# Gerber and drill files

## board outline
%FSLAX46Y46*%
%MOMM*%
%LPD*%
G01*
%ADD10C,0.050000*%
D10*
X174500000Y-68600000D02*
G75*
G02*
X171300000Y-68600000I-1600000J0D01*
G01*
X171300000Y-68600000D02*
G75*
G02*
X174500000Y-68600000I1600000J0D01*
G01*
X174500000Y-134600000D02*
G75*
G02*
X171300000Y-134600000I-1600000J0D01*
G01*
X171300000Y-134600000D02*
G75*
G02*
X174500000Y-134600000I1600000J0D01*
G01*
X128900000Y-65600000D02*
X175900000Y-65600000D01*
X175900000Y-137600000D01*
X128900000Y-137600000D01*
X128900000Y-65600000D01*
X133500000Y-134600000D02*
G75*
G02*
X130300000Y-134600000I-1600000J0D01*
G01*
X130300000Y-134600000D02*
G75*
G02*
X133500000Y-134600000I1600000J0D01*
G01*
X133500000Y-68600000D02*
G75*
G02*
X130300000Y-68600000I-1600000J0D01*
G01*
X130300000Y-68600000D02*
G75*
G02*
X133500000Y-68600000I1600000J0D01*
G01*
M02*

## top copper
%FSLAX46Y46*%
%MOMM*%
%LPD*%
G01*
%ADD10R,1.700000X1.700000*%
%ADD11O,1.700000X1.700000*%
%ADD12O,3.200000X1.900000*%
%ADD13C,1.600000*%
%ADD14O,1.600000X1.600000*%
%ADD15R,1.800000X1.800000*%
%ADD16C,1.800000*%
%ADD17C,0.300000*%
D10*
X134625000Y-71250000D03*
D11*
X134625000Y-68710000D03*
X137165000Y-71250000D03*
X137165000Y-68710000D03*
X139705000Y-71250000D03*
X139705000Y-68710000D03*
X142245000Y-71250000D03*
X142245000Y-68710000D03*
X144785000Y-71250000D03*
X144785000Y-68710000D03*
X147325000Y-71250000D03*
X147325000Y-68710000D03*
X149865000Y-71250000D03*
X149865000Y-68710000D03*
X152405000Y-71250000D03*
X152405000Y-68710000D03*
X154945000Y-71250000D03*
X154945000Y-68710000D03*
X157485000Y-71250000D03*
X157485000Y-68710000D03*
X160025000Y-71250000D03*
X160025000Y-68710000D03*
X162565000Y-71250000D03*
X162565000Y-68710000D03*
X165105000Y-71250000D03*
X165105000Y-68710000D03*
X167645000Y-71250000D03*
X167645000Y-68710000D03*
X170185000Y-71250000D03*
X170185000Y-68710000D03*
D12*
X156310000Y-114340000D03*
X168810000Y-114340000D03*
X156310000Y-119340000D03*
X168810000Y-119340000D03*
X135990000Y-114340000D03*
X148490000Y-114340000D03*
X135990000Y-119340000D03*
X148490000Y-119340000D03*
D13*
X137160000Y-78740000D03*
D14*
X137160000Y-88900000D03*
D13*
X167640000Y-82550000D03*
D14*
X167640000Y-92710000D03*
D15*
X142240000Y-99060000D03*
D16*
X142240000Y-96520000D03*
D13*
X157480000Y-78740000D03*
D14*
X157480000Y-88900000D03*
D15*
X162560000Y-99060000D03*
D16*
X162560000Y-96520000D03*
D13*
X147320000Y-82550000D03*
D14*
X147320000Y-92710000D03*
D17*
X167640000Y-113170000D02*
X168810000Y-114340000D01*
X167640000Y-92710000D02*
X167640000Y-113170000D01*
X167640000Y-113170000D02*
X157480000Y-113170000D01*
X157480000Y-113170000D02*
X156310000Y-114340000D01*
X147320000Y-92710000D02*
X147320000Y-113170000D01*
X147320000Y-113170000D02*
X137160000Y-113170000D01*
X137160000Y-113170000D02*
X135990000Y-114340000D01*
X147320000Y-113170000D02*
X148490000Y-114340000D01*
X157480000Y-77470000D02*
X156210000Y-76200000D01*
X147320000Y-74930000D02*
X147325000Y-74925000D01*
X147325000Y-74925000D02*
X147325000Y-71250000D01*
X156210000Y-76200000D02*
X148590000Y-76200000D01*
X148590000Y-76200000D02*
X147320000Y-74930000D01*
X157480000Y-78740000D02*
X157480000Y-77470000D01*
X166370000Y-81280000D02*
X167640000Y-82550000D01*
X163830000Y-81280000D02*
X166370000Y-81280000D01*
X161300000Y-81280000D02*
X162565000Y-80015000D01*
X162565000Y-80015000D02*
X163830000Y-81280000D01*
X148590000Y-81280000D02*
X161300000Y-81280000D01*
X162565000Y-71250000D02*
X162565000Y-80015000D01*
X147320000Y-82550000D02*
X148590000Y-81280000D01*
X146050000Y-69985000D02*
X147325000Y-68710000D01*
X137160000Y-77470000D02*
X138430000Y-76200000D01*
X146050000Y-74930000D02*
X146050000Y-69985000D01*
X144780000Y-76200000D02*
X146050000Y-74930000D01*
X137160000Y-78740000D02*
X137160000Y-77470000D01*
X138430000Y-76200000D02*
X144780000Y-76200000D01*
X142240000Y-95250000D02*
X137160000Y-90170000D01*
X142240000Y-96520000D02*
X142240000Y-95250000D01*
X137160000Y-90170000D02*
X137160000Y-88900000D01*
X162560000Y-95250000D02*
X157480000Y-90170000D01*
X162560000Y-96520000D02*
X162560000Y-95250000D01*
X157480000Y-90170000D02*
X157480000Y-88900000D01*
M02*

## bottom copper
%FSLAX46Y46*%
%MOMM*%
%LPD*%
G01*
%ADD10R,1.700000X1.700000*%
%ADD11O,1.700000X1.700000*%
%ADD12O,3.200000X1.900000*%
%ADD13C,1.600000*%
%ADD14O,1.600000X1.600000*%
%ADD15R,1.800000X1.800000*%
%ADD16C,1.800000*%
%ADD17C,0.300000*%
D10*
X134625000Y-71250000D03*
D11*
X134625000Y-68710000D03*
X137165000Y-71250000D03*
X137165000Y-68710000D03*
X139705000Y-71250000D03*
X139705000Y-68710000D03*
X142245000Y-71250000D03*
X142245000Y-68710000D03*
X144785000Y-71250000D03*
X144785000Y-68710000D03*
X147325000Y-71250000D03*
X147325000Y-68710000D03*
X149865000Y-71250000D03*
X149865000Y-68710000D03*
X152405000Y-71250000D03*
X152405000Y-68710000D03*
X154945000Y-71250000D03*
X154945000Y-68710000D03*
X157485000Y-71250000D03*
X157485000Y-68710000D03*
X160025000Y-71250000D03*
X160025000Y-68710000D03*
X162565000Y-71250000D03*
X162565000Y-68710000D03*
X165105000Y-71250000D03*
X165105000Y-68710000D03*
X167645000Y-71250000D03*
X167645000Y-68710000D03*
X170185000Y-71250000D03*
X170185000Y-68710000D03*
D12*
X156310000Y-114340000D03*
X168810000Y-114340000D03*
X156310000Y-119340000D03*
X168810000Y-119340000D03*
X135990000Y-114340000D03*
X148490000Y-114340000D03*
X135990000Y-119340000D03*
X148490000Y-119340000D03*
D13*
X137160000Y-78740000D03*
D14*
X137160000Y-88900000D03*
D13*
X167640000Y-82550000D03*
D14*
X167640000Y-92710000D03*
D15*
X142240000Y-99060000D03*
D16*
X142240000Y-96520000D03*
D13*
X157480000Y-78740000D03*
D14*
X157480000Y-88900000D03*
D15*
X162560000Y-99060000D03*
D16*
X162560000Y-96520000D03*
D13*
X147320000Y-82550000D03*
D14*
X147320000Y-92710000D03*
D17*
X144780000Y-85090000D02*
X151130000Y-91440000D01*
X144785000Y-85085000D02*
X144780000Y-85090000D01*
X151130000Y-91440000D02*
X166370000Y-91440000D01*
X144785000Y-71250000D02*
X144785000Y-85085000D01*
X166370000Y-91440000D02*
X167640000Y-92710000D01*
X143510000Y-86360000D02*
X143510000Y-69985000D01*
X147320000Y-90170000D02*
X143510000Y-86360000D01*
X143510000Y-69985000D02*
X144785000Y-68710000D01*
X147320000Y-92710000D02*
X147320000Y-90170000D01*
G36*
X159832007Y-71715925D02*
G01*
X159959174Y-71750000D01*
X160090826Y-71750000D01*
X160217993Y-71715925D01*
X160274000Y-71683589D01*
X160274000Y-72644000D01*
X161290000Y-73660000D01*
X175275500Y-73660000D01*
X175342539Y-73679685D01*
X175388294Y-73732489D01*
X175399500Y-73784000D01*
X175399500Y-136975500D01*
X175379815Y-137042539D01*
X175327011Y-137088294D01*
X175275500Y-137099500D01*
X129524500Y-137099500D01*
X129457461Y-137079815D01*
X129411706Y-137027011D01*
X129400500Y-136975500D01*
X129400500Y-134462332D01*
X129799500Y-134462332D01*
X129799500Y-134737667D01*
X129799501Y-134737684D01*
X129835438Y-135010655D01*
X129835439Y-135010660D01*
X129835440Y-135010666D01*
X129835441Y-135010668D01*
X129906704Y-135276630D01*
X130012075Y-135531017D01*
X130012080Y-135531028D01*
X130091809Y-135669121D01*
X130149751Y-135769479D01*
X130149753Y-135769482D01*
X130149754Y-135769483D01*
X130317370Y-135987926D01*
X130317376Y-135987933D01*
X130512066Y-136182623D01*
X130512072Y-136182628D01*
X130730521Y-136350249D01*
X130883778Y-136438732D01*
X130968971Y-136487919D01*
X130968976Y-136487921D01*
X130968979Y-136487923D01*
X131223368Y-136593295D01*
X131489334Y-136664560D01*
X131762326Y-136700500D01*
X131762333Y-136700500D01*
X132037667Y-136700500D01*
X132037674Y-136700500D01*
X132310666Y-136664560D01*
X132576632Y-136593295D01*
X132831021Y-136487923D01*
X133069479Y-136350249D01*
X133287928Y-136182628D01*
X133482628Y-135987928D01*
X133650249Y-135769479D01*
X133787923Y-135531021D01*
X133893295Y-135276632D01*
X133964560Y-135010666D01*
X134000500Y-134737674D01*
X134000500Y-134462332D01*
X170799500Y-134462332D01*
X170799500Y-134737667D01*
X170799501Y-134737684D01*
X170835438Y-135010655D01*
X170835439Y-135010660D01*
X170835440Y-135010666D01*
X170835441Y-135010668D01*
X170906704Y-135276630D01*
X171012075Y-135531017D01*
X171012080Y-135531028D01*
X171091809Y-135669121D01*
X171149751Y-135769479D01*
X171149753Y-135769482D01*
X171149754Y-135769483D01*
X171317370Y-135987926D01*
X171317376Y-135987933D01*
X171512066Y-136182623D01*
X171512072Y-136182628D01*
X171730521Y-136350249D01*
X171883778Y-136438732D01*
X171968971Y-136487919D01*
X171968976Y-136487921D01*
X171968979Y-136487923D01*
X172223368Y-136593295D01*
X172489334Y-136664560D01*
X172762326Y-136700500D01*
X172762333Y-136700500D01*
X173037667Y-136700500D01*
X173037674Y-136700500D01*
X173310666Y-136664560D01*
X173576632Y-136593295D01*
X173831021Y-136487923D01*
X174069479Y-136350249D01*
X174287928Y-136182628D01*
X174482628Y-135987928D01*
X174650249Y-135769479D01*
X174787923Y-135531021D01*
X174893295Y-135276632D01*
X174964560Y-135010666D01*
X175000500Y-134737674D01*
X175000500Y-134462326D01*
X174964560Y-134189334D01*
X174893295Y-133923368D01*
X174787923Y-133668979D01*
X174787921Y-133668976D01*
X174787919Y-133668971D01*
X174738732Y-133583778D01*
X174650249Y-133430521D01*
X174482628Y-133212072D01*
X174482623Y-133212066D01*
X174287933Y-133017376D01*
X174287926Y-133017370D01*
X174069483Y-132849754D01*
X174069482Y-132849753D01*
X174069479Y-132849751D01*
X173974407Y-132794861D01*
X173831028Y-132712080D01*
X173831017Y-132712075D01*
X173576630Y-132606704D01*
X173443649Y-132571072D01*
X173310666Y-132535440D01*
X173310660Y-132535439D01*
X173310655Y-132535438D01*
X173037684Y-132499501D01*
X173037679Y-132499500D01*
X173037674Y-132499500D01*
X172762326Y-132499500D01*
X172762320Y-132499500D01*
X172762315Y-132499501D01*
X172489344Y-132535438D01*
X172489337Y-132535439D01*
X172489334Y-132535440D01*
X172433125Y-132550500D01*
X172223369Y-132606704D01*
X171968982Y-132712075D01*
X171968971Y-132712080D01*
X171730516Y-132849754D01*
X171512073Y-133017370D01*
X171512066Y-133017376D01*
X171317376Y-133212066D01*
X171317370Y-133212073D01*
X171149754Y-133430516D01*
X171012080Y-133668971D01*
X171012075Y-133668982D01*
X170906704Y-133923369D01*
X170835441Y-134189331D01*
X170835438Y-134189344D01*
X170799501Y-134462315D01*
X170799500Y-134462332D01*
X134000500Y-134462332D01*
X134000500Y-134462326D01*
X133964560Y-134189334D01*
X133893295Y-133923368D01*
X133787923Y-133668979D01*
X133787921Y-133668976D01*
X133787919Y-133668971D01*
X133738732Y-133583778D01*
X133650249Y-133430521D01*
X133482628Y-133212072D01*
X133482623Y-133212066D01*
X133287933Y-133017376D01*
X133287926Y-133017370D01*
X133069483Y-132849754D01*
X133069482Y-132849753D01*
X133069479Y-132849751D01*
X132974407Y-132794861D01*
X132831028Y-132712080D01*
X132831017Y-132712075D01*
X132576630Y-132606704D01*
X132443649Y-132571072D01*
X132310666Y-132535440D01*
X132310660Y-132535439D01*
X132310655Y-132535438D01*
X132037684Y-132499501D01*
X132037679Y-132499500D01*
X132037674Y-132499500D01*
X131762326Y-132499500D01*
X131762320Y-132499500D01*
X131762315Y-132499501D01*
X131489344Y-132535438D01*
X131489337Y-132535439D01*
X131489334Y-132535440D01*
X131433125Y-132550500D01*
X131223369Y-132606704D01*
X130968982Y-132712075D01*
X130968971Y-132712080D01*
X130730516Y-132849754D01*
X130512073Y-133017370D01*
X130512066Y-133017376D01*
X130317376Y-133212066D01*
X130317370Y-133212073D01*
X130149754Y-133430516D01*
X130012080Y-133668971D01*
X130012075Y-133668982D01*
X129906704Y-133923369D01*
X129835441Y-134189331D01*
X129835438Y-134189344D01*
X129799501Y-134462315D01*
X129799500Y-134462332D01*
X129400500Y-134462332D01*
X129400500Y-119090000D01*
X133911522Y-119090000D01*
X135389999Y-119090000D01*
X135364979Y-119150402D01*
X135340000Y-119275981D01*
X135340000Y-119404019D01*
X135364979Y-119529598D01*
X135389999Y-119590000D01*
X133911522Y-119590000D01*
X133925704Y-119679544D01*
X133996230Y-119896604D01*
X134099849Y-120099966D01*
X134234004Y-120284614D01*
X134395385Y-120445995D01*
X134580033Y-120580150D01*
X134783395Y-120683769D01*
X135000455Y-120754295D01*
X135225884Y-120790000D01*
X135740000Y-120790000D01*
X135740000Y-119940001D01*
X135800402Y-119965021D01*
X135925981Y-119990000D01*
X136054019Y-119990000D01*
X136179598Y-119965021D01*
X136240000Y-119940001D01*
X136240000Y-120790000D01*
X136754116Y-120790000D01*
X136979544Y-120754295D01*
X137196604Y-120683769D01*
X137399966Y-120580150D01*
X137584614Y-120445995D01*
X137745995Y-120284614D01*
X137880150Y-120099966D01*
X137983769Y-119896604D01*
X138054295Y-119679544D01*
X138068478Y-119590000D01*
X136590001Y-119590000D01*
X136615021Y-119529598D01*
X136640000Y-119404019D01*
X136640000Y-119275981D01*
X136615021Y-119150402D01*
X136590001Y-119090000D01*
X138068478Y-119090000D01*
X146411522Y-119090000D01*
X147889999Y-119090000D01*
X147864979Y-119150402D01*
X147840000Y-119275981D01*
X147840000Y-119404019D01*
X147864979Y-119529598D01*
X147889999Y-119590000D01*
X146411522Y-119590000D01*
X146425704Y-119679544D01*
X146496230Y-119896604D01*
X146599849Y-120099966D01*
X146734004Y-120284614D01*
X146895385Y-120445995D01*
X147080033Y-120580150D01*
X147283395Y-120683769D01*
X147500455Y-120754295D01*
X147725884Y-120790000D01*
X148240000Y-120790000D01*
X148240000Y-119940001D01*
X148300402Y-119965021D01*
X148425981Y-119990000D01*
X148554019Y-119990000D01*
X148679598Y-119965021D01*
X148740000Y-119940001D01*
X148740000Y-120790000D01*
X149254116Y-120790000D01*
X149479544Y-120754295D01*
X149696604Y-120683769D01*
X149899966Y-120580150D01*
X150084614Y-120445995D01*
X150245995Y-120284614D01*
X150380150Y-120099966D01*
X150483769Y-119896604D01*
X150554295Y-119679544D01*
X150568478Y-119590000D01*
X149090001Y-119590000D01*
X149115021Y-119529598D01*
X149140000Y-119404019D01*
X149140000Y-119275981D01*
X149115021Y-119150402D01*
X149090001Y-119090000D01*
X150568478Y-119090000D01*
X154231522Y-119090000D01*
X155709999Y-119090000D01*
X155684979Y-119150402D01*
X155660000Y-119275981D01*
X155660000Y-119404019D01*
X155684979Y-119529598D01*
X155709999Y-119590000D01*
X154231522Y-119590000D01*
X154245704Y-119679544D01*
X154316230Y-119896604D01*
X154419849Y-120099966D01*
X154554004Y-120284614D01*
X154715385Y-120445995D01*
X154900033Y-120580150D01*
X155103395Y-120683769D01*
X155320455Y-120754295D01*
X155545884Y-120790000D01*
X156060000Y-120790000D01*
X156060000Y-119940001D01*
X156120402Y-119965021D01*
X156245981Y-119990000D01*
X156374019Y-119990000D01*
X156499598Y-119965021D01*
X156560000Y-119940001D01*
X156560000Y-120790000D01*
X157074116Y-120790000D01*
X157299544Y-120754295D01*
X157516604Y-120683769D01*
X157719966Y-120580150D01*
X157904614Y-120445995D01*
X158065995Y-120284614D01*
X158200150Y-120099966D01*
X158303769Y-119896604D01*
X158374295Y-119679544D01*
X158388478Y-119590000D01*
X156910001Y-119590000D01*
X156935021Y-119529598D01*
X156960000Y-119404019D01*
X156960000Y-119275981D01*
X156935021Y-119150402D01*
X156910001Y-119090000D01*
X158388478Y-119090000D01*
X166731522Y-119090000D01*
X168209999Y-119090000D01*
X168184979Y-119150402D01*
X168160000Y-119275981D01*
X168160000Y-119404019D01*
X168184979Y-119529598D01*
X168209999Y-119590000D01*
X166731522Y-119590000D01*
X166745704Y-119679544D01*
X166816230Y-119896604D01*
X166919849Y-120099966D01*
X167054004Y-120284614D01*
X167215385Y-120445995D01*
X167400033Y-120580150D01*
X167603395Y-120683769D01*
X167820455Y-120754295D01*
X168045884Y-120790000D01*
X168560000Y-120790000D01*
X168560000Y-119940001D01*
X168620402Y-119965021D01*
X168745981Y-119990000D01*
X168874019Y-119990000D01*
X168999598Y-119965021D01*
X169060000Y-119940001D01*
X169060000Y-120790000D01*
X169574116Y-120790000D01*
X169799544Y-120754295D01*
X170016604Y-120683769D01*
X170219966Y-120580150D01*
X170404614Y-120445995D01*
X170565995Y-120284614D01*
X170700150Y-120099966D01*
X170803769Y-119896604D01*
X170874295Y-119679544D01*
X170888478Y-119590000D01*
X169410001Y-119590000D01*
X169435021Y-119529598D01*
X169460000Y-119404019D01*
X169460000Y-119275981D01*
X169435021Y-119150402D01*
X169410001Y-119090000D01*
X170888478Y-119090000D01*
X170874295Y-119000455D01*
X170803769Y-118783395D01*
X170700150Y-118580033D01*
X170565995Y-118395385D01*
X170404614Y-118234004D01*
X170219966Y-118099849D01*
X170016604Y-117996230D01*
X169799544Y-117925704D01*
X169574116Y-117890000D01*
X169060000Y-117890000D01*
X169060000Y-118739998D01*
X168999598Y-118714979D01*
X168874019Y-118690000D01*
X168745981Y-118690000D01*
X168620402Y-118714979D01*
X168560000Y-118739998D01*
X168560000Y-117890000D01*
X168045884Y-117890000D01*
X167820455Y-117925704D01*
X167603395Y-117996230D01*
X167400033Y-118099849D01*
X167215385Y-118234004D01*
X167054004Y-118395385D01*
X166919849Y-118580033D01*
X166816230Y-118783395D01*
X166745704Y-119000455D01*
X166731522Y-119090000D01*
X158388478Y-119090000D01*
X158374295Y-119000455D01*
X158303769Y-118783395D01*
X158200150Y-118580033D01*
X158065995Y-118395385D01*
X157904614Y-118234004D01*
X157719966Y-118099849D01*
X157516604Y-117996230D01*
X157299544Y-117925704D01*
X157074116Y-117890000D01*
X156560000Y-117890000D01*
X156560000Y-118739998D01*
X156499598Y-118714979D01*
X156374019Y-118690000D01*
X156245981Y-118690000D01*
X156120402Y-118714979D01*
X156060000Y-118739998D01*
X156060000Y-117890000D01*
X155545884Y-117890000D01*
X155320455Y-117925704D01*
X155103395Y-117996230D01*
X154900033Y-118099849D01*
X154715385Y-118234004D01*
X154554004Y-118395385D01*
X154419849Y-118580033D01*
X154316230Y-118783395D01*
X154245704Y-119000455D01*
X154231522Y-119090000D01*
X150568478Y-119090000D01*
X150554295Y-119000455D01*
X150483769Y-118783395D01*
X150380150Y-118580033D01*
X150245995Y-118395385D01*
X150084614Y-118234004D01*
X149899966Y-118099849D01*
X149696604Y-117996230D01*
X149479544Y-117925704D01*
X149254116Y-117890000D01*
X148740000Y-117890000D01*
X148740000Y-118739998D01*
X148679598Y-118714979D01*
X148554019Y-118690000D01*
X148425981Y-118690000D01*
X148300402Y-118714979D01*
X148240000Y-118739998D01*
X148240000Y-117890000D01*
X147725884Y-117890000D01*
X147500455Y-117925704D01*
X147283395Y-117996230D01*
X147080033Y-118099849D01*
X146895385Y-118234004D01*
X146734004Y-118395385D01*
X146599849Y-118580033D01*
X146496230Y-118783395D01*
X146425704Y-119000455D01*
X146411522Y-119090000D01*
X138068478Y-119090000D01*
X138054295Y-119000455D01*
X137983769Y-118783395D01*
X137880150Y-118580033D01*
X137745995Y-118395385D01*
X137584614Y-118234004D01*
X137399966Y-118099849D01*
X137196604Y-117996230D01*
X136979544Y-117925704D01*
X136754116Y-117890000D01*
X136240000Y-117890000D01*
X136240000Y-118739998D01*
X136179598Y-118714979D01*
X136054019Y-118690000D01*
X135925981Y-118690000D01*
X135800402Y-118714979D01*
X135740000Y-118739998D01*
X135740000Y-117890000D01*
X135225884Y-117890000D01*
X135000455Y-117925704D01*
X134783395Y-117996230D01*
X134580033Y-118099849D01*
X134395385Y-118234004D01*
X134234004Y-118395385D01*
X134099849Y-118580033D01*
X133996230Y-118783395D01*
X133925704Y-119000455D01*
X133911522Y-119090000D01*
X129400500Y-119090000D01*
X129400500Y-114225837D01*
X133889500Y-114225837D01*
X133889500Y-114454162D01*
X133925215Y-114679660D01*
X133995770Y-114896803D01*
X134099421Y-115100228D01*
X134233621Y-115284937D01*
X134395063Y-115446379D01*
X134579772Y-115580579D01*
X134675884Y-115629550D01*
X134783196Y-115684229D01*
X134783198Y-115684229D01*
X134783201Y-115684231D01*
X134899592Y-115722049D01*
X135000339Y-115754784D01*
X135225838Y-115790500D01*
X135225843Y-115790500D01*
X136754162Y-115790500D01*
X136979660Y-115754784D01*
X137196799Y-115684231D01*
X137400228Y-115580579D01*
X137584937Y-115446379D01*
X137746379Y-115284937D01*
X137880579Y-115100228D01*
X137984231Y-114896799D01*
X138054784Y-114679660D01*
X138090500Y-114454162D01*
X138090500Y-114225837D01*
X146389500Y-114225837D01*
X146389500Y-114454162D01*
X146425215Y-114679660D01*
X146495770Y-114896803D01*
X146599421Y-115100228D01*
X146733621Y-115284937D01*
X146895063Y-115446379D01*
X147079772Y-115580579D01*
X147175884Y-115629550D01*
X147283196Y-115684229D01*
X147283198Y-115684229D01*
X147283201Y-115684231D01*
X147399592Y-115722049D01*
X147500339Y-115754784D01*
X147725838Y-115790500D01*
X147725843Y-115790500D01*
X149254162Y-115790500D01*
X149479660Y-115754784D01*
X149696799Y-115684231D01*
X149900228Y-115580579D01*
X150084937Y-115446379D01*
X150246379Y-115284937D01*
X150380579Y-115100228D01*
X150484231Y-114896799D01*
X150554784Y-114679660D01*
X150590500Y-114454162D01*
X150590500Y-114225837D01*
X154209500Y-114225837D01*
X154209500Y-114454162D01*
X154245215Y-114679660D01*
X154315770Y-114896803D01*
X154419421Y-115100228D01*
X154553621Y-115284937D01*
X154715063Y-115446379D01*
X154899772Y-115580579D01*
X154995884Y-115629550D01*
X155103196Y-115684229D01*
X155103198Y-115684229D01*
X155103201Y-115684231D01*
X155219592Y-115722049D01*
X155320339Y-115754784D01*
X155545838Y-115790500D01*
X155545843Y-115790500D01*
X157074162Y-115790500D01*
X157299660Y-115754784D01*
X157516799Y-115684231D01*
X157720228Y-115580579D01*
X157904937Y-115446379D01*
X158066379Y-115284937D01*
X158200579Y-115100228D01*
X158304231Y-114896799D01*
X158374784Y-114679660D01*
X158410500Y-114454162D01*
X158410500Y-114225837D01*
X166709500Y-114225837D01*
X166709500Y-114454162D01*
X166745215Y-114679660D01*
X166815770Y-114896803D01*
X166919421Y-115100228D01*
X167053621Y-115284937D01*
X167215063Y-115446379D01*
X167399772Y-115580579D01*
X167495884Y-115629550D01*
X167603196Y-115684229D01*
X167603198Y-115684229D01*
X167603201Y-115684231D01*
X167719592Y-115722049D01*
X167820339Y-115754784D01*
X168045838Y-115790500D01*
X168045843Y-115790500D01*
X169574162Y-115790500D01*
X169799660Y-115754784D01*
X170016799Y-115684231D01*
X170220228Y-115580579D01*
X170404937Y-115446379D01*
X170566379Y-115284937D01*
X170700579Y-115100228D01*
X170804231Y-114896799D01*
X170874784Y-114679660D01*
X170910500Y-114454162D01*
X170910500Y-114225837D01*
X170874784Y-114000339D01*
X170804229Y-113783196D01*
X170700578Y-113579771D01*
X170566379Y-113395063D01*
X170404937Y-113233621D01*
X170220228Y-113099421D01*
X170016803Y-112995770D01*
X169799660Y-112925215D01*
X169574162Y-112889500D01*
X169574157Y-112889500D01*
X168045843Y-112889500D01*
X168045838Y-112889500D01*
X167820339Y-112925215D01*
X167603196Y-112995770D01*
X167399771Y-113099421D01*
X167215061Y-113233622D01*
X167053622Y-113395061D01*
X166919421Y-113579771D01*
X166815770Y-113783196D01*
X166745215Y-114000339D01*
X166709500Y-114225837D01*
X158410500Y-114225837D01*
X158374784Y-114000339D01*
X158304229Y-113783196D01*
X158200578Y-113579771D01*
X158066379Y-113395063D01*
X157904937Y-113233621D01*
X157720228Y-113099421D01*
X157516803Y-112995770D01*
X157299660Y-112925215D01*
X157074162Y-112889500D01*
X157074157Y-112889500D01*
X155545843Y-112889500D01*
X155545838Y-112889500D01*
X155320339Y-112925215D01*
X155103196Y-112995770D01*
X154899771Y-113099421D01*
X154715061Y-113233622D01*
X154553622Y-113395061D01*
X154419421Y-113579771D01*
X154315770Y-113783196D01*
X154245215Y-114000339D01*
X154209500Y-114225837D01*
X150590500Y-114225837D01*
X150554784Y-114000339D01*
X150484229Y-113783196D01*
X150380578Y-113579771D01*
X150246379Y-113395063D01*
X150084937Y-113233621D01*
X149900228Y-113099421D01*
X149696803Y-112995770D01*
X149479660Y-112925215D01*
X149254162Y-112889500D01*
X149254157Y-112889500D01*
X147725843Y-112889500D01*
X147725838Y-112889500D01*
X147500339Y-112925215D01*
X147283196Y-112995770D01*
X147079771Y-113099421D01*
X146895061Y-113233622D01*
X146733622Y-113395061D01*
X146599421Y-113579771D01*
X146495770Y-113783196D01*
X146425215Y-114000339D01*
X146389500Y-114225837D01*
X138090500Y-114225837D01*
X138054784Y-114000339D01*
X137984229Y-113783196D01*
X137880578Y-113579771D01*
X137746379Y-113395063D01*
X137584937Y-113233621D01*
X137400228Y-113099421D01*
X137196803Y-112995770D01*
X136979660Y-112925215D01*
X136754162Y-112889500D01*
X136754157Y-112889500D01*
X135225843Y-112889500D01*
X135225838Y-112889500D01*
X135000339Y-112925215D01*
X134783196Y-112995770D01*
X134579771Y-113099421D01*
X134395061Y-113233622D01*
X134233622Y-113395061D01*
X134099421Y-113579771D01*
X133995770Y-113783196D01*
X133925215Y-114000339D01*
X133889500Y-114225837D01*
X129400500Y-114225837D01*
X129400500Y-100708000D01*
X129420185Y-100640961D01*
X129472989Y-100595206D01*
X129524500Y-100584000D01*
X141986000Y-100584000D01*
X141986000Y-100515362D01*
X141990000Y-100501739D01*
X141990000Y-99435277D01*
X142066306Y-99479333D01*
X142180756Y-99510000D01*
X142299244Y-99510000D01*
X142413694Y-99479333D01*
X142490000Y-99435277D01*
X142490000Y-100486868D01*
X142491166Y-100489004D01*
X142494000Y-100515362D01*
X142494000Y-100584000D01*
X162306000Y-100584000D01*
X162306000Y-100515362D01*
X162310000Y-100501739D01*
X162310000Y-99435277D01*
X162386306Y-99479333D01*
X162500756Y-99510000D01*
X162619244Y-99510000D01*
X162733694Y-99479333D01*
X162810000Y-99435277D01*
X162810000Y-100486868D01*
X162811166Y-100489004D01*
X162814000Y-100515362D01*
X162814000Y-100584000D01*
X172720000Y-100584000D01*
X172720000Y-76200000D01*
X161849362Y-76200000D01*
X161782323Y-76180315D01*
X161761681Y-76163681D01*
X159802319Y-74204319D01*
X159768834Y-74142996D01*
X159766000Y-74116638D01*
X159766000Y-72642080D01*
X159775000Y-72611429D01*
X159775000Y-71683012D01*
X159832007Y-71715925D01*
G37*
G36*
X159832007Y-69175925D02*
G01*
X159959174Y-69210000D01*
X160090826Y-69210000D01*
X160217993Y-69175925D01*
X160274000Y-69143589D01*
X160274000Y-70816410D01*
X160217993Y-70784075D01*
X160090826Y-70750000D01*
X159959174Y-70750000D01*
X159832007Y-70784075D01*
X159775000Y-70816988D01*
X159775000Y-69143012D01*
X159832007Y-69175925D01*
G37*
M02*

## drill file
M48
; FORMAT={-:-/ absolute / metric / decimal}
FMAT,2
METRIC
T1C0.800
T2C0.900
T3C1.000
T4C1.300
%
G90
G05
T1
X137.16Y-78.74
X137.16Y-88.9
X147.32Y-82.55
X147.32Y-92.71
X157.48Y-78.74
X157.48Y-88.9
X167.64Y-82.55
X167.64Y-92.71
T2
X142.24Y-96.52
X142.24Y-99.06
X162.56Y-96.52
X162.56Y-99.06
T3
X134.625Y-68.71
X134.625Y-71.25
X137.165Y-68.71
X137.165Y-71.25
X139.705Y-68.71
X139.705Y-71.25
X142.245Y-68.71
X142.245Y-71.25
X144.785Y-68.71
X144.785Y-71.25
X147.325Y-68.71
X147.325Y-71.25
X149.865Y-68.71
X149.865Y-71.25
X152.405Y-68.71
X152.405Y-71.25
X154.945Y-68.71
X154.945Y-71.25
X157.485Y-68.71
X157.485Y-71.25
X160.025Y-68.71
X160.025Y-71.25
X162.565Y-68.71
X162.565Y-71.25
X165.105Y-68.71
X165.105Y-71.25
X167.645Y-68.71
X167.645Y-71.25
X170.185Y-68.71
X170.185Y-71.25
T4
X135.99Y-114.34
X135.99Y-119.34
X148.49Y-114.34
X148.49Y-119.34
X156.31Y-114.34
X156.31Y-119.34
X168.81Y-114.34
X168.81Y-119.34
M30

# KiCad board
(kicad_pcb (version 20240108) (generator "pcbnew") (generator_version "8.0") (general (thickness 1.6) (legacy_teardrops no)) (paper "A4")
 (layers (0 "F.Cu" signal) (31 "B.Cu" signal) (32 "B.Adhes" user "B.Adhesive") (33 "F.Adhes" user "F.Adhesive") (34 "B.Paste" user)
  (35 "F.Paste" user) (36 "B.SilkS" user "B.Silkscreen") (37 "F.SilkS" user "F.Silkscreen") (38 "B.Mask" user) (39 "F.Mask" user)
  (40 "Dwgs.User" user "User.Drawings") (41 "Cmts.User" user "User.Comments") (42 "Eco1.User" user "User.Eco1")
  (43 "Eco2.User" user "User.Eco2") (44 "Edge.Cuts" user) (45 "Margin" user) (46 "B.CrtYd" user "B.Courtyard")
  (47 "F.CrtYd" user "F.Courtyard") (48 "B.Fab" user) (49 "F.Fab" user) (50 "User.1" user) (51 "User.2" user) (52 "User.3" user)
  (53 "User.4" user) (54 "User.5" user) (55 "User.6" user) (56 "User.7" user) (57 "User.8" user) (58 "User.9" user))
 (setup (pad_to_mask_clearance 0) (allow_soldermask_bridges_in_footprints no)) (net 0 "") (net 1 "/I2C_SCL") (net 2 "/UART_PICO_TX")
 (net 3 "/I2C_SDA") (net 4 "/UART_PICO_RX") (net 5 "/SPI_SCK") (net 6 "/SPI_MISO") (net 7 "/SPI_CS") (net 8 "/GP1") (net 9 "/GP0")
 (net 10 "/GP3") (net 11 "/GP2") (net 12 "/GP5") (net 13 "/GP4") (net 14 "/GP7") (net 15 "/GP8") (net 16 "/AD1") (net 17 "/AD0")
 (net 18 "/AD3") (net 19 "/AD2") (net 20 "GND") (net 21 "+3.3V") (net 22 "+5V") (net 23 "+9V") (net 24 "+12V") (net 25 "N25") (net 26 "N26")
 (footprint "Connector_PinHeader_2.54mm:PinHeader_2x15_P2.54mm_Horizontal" (layer "F.Cu") (at 134.625 71.25 90)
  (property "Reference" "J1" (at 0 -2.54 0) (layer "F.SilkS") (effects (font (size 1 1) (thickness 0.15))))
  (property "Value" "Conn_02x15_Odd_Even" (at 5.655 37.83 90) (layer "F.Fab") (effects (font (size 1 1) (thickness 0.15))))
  (pad "1" thru_hole rect (at 0 0 90) (size 1.7 1.7) (drill 1) (layers "*.Cu" "*.Mask") (remove_unused_layers no) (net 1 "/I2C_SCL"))
  (pad "2" thru_hole oval (at 2.54 0 90) (size 1.7 1.7) (drill 1) (layers "*.Cu" "*.Mask") (remove_unused_layers no) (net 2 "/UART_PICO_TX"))
  (pad "3" thru_hole oval (at 0 2.54 90) (size 1.7 1.7) (drill 1) (layers "*.Cu" "*.Mask") (remove_unused_layers no) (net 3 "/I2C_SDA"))
  (pad "4" thru_hole oval (at 2.54 2.54 90) (size 1.7 1.7) (drill 1) (layers "*.Cu" "*.Mask") (remove_unused_layers no)
   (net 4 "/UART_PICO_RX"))
  (pad "5" thru_hole oval (at 0 5.08 90) (size 1.7 1.7) (drill 1) (layers "*.Cu" "*.Mask") (remove_unused_layers no) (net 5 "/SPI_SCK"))
  (pad "6" thru_hole oval (at 2.54 5.08 90) (size 1.7 1.7) (drill 1) (layers "*.Cu" "*.Mask") (remove_unused_layers no) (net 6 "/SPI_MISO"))
  (pad "7" thru_hole oval (at 0 7.62 90) (size 1.7 1.7) (drill 1) (layers "*.Cu" "*.Mask") (remove_unused_layers no) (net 6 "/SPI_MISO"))
  (pad "8" thru_hole oval (at 2.54 7.62 90) (size 1.7 1.7) (drill 1) (layers "*.Cu" "*.Mask") (remove_unused_layers no) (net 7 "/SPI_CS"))
  (pad "9" thru_hole oval (at 0 10.16 90) (size 1.7 1.7) (drill 1) (layers "*.Cu" "*.Mask") (remove_unused_layers no) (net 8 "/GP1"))
  (pad "10" thru_hole oval (at 2.54 10.16 90) (size 1.7 1.7) (drill 1) (layers "*.Cu" "*.Mask") (remove_unused_layers no) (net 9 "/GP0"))
  (pad "11" thru_hole oval (at 0 12.7 90) (size 1.7 1.7) (drill 1) (layers "*.Cu" "*.Mask") (remove_unused_layers no) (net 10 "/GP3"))
  (pad "12" thru_hole oval (at 2.54 12.7 90) (size 1.7 1.7) (drill 1) (layers "*.Cu" "*.Mask") (remove_unused_layers no) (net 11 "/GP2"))
  (pad "13" thru_hole oval (at 0 15.24 90) (size 1.7 1.7) (drill 1) (layers "*.Cu" "*.Mask") (remove_unused_layers no) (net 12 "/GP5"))
  (pad "14" thru_hole oval (at 2.54 15.24 90) (size 1.7 1.7) (drill 1) (layers "*.Cu" "*.Mask") (remove_unused_layers no) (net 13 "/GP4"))
  (pad "15" thru_hole oval (at 0 17.78 90) (size 1.7 1.7) (drill 1) (layers "*.Cu" "*.Mask") (remove_unused_layers no) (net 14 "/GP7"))
  (pad "16" thru_hole oval (at 2.54 17.78 90) (size 1.7 1.7) (drill 1) (layers "*.Cu" "*.Mask") (remove_unused_layers no) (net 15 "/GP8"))
  (pad "17" thru_hole oval (at 0 20.32 90) (size 1.7 1.7) (drill 1) (layers "*.Cu" "*.Mask") (remove_unused_layers no) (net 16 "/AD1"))
  (pad "18" thru_hole oval (at 2.54 20.32 90) (size 1.7 1.7) (drill 1) (layers "*.Cu" "*.Mask") (remove_unused_layers no) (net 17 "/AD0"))
  (pad "19" thru_hole oval (at 0 22.86 90) (size 1.7 1.7) (drill 1) (layers "*.Cu" "*.Mask") (remove_unused_layers no) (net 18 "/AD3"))
  (pad "20" thru_hole oval (at 2.54 22.86 90) (size 1.7 1.7) (drill 1) (layers "*.Cu" "*.Mask") (remove_unused_layers no) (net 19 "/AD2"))
  (pad "21" thru_hole oval (at 0 25.4 90) (size 1.7 1.7) (drill 1) (layers "*.Cu" "*.Mask") (remove_unused_layers no) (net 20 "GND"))
  (pad "22" thru_hole oval (at 2.54 25.4 90) (size 1.7 1.7) (drill 1) (layers "*.Cu" "*.Mask") (remove_unused_layers no) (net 20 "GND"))
  (pad "23" thru_hole oval (at 0 27.94 90) (size 1.7 1.7) (drill 1) (layers "*.Cu" "*.Mask") (remove_unused_layers no) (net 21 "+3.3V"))
  (pad "24" thru_hole oval (at 2.54 27.94 90) (size 1.7 1.7) (drill 1) (layers "*.Cu" "*.Mask") (remove_unused_layers no) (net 21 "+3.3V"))
  (pad "25" thru_hole oval (at 0 30.48 90) (size 1.7 1.7) (drill 1) (layers "*.Cu" "*.Mask") (remove_unused_layers no) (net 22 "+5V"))
  (pad "26" thru_hole oval (at 2.54 30.48 90) (size 1.7 1.7) (drill 1) (layers "*.Cu" "*.Mask") (remove_unused_layers no) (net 22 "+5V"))
  (pad "27" thru_hole oval (at 0 33.02 90) (size 1.7 1.7) (drill 1) (layers "*.Cu" "*.Mask") (remove_unused_layers no) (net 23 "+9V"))
  (pad "28" thru_hole oval (at 2.54 33.02 90) (size 1.7 1.7) (drill 1) (layers "*.Cu" "*.Mask") (remove_unused_layers no) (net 23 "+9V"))
  (pad "29" thru_hole oval (at 0 35.56 90) (size 1.7 1.7) (drill 1) (layers "*.Cu" "*.Mask") (remove_unused_layers no) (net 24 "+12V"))
  (pad "30" thru_hole oval (at 2.54 35.56 90) (size 1.7 1.7) (drill 1) (layers "*.Cu" "*.Mask") (remove_unused_layers no) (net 24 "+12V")))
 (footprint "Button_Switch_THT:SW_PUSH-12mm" (layer "F.Cu") (at 156.31 114.34)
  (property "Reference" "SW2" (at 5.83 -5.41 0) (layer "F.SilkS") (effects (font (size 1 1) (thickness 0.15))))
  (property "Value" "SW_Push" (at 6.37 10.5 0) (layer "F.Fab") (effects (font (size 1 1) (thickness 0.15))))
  (pad "1" thru_hole oval (at 0 0) (size 3.2 1.9) (drill 1.3) (layers "*.Cu" "*.Mask") (remove_unused_layers no) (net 8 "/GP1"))
  (pad "1" thru_hole oval (at 12.5 0) (size 3.2 1.9) (drill 1.3) (layers "*.Cu" "*.Mask") (remove_unused_layers no) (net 8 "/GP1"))
  (pad "2" thru_hole oval (at 0 5) (size 3.2 1.9) (drill 1.3) (layers "*.Cu" "*.Mask") (remove_unused_layers no) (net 20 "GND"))
  (pad "2" thru_hole oval (at 12.5 5) (size 3.2 1.9) (drill 1.3) (layers "*.Cu" "*.Mask") (remove_unused_layers no) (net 20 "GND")))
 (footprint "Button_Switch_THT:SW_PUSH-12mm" (layer "F.Cu") (at 135.99 114.34)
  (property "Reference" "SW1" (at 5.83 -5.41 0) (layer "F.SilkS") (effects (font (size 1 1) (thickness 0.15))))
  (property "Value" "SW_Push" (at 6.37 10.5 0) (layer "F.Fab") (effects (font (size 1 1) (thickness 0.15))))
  (pad "1" thru_hole oval (at 0 0) (size 3.2 1.9) (drill 1.3) (layers "*.Cu" "*.Mask") (remove_unused_layers no) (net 9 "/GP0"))
  (pad "1" thru_hole oval (at 12.5 0) (size 3.2 1.9) (drill 1.3) (layers "*.Cu" "*.Mask") (remove_unused_layers no) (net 9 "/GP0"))
  (pad "2" thru_hole oval (at 0 5) (size 3.2 1.9) (drill 1.3) (layers "*.Cu" "*.Mask") (remove_unused_layers no) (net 20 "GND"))
  (pad "2" thru_hole oval (at 12.5 5) (size 3.2 1.9) (drill 1.3) (layers "*.Cu" "*.Mask") (remove_unused_layers no) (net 20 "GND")))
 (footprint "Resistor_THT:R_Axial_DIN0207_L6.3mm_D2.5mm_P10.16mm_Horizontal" (layer "F.Cu") (at 137.16 78.74 -90)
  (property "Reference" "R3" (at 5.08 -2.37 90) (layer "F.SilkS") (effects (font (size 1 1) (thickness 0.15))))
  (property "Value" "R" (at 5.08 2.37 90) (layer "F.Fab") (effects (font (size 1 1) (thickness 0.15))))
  (pad "1" thru_hole circle (at 0 0 270) (size 1.6 1.6) (drill 0.8) (layers "*.Cu" "*.Mask") (remove_unused_layers no) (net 11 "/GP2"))
  (pad "2" thru_hole oval (at 10.16 0 270) (size 1.6 1.6) (drill 0.8) (layers "*.Cu" "*.Mask") (remove_unused_layers no) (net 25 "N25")))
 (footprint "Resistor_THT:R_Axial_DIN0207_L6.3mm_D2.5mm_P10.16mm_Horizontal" (layer "F.Cu") (at 167.64 82.55 -90)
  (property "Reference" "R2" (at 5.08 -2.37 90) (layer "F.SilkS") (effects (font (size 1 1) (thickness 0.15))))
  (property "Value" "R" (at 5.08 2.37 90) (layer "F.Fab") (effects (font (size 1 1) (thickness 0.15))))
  (pad "1" thru_hole circle (at 0 0 270) (size 1.6 1.6) (drill 0.8) (layers "*.Cu" "*.Mask") (remove_unused_layers no) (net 21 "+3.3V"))
  (pad "2" thru_hole oval (at 10.16 0 270) (size 1.6 1.6) (drill 0.8) (layers "*.Cu" "*.Mask") (remove_unused_layers no) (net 8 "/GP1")))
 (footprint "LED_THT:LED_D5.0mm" (layer "F.Cu") (at 142.24 99.06 90)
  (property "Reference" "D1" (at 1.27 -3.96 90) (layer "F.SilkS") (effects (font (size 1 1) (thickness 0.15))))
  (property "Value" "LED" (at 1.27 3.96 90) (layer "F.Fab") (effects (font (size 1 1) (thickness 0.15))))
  (pad "1" thru_hole rect (at 0 0 90) (size 1.8 1.8) (drill 0.9) (layers "*.Cu" "*.Mask") (remove_unused_layers no) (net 20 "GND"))
  (pad "2" thru_hole circle (at 2.54 0 90) (size 1.8 1.8) (drill 0.9) (layers "*.Cu" "*.Mask") (remove_unused_layers no) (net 25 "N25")))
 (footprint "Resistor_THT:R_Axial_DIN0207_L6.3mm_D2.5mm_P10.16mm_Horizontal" (layer "F.Cu") (at 157.48 78.74 -90)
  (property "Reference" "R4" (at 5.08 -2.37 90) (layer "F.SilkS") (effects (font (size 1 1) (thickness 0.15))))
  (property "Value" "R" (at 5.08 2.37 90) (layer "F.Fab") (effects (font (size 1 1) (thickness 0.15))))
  (pad "1" thru_hole circle (at 0 0 270) (size 1.6 1.6) (drill 0.8) (layers "*.Cu" "*.Mask") (remove_unused_layers no) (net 10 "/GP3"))
  (pad "2" thru_hole oval (at 10.16 0 270) (size 1.6 1.6) (drill 0.8) (layers "*.Cu" "*.Mask") (remove_unused_layers no) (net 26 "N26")))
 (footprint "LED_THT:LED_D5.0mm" (layer "F.Cu") (at 162.56 99.06 90)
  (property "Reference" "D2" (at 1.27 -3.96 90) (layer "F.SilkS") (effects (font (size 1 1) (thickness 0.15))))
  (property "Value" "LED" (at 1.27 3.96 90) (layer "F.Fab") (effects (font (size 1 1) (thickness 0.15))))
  (pad "1" thru_hole rect (at 0 0 90) (size 1.8 1.8) (drill 0.9) (layers "*.Cu" "*.Mask") (remove_unused_layers no) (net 20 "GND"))
  (pad "2" thru_hole circle (at 2.54 0 90) (size 1.8 1.8) (drill 0.9) (layers "*.Cu" "*.Mask") (remove_unused_layers no) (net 26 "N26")))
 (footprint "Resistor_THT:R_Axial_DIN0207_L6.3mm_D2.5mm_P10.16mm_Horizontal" (layer "F.Cu") (at 147.32 82.55 -90)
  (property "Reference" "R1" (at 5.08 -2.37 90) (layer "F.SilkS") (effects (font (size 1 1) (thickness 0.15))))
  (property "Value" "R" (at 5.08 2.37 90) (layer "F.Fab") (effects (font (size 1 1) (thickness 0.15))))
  (pad "1" thru_hole circle (at 0 0 270) (size 1.6 1.6) (drill 0.8) (layers "*.Cu" "*.Mask") (remove_unused_layers no) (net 21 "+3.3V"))
  (pad "2" thru_hole oval (at 10.16 0 270) (size 1.6 1.6) (drill 0.8) (layers "*.Cu" "*.Mask") (remove_unused_layers no) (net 9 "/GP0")))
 (gr_circle (center 172.9 68.6) (end 172.9 70.2) (stroke (width 0.05) (type default)) (fill none) (layer "Edge.Cuts"))
 (gr_circle (center 172.9 134.6) (end 171.3 134.6) (stroke (width 0.05) (type default)) (fill none) (layer "Edge.Cuts"))
 (gr_rect (start 128.9 65.6) (end 175.9 137.6) (stroke (width 0.05) (type default)) (fill none) (layer "Edge.Cuts"))
 (gr_circle (center 131.9 134.6) (end 131.9 133) (stroke (width 0.05) (type default)) (fill none) (layer "Edge.Cuts"))
 (gr_circle (center 131.9 68.6) (end 133.5 68.6) (stroke (width 0.05) (type default)) (fill none) (layer "Edge.Cuts"))
 (segment (start 167.64 113.17) (end 168.81 114.34) (width 0.3) (layer "F.Cu") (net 8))
 (segment (start 167.64 92.71) (end 167.64 113.17) (width 0.3) (layer "F.Cu") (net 8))
 (segment (start 167.64 113.17) (end 157.48 113.17) (width 0.3) (layer "F.Cu") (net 8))
 (segment (start 157.48 113.17) (end 156.31 114.34) (width 0.3) (layer "F.Cu") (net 8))
 (segment (start 144.78 85.09) (end 151.13 91.44) (width 0.3) (layer "B.Cu") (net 8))
 (segment (start 144.785 85.085) (end 144.78 85.09) (width 0.3) (layer "B.Cu") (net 8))
 (segment (start 151.13 91.44) (end 166.37 91.44) (width 0.3) (layer "B.Cu") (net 8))
 (segment (start 144.785 71.25) (end 144.785 85.085) (width 0.3) (layer "B.Cu") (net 8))
 (segment (start 166.37 91.44) (end 167.64 92.71) (width 0.3) (layer "B.Cu") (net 8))
 (segment (start 147.32 92.71) (end 147.32 113.17) (width 0.3) (layer "F.Cu") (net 9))
 (segment (start 147.32 113.17) (end 137.16 113.17) (width 0.3) (layer "F.Cu") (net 9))
 (segment (start 137.16 113.17) (end 135.99 114.34) (width 0.3) (layer "F.Cu") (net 9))
 (segment (start 147.32 113.17) (end 148.49 114.34) (width 0.3) (layer "F.Cu") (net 9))
 (segment (start 143.51 86.36) (end 143.51 69.985) (width 0.3) (layer "B.Cu") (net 9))
 (segment (start 147.32 90.17) (end 143.51 86.36) (width 0.3) (layer "B.Cu") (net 9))
 (segment (start 143.51 69.985) (end 144.785 68.71) (width 0.3) (layer "B.Cu") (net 9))
 (segment (start 147.32 92.71) (end 147.32 90.17) (width 0.3) (layer "B.Cu") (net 9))
 (segment (start 157.48 77.47) (end 156.21 76.2) (width 0.3) (layer "F.Cu") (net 10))
 (segment (start 147.32 74.93) (end 147.325 74.925) (width 0.3) (layer "F.Cu") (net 10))
 (segment (start 147.325 74.925) (end 147.325 71.25) (width 0.3) (layer "F.Cu") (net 10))
 (segment (start 156.21 76.2) (end 148.59 76.2) (width 0.3) (layer "F.Cu") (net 10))
 (segment (start 148.59 76.2) (end 147.32 74.93) (width 0.3) (layer "F.Cu") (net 10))
 (segment (start 157.48 78.74) (end 157.48 77.47) (width 0.3) (layer "F.Cu") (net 10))
 (segment (start 166.37 81.28) (end 167.64 82.55) (width 0.3) (layer "F.Cu") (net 21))
 (segment (start 163.83 81.28) (end 166.37 81.28) (width 0.3) (layer "F.Cu") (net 21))
 (segment (start 161.3 81.28) (end 162.565 80.015) (width 0.3) (layer "F.Cu") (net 21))
 (segment (start 162.565 80.015) (end 163.83 81.28) (width 0.3) (layer "F.Cu") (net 21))
 (segment (start 148.59 81.28) (end 161.3 81.28) (width 0.3) (layer "F.Cu") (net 21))
 (segment (start 162.565 71.25) (end 162.565 80.015) (width 0.3) (layer "F.Cu") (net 21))
 (segment (start 147.32 82.55) (end 148.59 81.28) (width 0.3) (layer "F.Cu") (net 21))
 (segment (start 146.05 69.985) (end 147.325 68.71) (width 0.3) (layer "F.Cu") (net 11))
 (segment (start 137.16 77.47) (end 138.43 76.2) (width 0.3) (layer "F.Cu") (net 11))
 (segment (start 146.05 74.93) (end 146.05 69.985) (width 0.3) (layer "F.Cu") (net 11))
 (segment (start 144.78 76.2) (end 146.05 74.93) (width 0.3) (layer "F.Cu") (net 11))
 (segment (start 137.16 78.74) (end 137.16 77.47) (width 0.3) (layer "F.Cu") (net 11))
 (segment (start 138.43 76.2) (end 144.78 76.2) (width 0.3) (layer "F.Cu") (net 11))
 (segment (start 142.24 95.25) (end 137.16 90.17) (width 0.3) (layer "F.Cu") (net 25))
 (segment (start 142.24 96.52) (end 142.24 95.25) (width 0.3) (layer "F.Cu") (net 25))
 (segment (start 137.16 90.17) (end 137.16 88.9) (width 0.3) (layer "F.Cu") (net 25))
 (segment (start 162.56 95.25) (end 157.48 90.17) (width 0.3) (layer "F.Cu") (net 26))
 (segment (start 162.56 96.52) (end 162.56 95.25) (width 0.3) (layer "F.Cu") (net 26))
 (segment (start 157.48 90.17) (end 157.48 88.9) (width 0.3) (layer "F.Cu") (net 26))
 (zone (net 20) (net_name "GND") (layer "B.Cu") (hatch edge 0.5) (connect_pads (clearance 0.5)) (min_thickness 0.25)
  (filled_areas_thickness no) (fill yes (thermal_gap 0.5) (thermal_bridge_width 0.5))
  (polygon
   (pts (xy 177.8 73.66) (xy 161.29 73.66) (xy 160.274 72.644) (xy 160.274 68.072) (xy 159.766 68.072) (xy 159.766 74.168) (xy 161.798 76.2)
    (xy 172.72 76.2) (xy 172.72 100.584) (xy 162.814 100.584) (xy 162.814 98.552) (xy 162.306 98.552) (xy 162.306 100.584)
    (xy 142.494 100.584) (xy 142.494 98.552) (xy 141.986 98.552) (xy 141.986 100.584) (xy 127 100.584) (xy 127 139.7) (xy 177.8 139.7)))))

